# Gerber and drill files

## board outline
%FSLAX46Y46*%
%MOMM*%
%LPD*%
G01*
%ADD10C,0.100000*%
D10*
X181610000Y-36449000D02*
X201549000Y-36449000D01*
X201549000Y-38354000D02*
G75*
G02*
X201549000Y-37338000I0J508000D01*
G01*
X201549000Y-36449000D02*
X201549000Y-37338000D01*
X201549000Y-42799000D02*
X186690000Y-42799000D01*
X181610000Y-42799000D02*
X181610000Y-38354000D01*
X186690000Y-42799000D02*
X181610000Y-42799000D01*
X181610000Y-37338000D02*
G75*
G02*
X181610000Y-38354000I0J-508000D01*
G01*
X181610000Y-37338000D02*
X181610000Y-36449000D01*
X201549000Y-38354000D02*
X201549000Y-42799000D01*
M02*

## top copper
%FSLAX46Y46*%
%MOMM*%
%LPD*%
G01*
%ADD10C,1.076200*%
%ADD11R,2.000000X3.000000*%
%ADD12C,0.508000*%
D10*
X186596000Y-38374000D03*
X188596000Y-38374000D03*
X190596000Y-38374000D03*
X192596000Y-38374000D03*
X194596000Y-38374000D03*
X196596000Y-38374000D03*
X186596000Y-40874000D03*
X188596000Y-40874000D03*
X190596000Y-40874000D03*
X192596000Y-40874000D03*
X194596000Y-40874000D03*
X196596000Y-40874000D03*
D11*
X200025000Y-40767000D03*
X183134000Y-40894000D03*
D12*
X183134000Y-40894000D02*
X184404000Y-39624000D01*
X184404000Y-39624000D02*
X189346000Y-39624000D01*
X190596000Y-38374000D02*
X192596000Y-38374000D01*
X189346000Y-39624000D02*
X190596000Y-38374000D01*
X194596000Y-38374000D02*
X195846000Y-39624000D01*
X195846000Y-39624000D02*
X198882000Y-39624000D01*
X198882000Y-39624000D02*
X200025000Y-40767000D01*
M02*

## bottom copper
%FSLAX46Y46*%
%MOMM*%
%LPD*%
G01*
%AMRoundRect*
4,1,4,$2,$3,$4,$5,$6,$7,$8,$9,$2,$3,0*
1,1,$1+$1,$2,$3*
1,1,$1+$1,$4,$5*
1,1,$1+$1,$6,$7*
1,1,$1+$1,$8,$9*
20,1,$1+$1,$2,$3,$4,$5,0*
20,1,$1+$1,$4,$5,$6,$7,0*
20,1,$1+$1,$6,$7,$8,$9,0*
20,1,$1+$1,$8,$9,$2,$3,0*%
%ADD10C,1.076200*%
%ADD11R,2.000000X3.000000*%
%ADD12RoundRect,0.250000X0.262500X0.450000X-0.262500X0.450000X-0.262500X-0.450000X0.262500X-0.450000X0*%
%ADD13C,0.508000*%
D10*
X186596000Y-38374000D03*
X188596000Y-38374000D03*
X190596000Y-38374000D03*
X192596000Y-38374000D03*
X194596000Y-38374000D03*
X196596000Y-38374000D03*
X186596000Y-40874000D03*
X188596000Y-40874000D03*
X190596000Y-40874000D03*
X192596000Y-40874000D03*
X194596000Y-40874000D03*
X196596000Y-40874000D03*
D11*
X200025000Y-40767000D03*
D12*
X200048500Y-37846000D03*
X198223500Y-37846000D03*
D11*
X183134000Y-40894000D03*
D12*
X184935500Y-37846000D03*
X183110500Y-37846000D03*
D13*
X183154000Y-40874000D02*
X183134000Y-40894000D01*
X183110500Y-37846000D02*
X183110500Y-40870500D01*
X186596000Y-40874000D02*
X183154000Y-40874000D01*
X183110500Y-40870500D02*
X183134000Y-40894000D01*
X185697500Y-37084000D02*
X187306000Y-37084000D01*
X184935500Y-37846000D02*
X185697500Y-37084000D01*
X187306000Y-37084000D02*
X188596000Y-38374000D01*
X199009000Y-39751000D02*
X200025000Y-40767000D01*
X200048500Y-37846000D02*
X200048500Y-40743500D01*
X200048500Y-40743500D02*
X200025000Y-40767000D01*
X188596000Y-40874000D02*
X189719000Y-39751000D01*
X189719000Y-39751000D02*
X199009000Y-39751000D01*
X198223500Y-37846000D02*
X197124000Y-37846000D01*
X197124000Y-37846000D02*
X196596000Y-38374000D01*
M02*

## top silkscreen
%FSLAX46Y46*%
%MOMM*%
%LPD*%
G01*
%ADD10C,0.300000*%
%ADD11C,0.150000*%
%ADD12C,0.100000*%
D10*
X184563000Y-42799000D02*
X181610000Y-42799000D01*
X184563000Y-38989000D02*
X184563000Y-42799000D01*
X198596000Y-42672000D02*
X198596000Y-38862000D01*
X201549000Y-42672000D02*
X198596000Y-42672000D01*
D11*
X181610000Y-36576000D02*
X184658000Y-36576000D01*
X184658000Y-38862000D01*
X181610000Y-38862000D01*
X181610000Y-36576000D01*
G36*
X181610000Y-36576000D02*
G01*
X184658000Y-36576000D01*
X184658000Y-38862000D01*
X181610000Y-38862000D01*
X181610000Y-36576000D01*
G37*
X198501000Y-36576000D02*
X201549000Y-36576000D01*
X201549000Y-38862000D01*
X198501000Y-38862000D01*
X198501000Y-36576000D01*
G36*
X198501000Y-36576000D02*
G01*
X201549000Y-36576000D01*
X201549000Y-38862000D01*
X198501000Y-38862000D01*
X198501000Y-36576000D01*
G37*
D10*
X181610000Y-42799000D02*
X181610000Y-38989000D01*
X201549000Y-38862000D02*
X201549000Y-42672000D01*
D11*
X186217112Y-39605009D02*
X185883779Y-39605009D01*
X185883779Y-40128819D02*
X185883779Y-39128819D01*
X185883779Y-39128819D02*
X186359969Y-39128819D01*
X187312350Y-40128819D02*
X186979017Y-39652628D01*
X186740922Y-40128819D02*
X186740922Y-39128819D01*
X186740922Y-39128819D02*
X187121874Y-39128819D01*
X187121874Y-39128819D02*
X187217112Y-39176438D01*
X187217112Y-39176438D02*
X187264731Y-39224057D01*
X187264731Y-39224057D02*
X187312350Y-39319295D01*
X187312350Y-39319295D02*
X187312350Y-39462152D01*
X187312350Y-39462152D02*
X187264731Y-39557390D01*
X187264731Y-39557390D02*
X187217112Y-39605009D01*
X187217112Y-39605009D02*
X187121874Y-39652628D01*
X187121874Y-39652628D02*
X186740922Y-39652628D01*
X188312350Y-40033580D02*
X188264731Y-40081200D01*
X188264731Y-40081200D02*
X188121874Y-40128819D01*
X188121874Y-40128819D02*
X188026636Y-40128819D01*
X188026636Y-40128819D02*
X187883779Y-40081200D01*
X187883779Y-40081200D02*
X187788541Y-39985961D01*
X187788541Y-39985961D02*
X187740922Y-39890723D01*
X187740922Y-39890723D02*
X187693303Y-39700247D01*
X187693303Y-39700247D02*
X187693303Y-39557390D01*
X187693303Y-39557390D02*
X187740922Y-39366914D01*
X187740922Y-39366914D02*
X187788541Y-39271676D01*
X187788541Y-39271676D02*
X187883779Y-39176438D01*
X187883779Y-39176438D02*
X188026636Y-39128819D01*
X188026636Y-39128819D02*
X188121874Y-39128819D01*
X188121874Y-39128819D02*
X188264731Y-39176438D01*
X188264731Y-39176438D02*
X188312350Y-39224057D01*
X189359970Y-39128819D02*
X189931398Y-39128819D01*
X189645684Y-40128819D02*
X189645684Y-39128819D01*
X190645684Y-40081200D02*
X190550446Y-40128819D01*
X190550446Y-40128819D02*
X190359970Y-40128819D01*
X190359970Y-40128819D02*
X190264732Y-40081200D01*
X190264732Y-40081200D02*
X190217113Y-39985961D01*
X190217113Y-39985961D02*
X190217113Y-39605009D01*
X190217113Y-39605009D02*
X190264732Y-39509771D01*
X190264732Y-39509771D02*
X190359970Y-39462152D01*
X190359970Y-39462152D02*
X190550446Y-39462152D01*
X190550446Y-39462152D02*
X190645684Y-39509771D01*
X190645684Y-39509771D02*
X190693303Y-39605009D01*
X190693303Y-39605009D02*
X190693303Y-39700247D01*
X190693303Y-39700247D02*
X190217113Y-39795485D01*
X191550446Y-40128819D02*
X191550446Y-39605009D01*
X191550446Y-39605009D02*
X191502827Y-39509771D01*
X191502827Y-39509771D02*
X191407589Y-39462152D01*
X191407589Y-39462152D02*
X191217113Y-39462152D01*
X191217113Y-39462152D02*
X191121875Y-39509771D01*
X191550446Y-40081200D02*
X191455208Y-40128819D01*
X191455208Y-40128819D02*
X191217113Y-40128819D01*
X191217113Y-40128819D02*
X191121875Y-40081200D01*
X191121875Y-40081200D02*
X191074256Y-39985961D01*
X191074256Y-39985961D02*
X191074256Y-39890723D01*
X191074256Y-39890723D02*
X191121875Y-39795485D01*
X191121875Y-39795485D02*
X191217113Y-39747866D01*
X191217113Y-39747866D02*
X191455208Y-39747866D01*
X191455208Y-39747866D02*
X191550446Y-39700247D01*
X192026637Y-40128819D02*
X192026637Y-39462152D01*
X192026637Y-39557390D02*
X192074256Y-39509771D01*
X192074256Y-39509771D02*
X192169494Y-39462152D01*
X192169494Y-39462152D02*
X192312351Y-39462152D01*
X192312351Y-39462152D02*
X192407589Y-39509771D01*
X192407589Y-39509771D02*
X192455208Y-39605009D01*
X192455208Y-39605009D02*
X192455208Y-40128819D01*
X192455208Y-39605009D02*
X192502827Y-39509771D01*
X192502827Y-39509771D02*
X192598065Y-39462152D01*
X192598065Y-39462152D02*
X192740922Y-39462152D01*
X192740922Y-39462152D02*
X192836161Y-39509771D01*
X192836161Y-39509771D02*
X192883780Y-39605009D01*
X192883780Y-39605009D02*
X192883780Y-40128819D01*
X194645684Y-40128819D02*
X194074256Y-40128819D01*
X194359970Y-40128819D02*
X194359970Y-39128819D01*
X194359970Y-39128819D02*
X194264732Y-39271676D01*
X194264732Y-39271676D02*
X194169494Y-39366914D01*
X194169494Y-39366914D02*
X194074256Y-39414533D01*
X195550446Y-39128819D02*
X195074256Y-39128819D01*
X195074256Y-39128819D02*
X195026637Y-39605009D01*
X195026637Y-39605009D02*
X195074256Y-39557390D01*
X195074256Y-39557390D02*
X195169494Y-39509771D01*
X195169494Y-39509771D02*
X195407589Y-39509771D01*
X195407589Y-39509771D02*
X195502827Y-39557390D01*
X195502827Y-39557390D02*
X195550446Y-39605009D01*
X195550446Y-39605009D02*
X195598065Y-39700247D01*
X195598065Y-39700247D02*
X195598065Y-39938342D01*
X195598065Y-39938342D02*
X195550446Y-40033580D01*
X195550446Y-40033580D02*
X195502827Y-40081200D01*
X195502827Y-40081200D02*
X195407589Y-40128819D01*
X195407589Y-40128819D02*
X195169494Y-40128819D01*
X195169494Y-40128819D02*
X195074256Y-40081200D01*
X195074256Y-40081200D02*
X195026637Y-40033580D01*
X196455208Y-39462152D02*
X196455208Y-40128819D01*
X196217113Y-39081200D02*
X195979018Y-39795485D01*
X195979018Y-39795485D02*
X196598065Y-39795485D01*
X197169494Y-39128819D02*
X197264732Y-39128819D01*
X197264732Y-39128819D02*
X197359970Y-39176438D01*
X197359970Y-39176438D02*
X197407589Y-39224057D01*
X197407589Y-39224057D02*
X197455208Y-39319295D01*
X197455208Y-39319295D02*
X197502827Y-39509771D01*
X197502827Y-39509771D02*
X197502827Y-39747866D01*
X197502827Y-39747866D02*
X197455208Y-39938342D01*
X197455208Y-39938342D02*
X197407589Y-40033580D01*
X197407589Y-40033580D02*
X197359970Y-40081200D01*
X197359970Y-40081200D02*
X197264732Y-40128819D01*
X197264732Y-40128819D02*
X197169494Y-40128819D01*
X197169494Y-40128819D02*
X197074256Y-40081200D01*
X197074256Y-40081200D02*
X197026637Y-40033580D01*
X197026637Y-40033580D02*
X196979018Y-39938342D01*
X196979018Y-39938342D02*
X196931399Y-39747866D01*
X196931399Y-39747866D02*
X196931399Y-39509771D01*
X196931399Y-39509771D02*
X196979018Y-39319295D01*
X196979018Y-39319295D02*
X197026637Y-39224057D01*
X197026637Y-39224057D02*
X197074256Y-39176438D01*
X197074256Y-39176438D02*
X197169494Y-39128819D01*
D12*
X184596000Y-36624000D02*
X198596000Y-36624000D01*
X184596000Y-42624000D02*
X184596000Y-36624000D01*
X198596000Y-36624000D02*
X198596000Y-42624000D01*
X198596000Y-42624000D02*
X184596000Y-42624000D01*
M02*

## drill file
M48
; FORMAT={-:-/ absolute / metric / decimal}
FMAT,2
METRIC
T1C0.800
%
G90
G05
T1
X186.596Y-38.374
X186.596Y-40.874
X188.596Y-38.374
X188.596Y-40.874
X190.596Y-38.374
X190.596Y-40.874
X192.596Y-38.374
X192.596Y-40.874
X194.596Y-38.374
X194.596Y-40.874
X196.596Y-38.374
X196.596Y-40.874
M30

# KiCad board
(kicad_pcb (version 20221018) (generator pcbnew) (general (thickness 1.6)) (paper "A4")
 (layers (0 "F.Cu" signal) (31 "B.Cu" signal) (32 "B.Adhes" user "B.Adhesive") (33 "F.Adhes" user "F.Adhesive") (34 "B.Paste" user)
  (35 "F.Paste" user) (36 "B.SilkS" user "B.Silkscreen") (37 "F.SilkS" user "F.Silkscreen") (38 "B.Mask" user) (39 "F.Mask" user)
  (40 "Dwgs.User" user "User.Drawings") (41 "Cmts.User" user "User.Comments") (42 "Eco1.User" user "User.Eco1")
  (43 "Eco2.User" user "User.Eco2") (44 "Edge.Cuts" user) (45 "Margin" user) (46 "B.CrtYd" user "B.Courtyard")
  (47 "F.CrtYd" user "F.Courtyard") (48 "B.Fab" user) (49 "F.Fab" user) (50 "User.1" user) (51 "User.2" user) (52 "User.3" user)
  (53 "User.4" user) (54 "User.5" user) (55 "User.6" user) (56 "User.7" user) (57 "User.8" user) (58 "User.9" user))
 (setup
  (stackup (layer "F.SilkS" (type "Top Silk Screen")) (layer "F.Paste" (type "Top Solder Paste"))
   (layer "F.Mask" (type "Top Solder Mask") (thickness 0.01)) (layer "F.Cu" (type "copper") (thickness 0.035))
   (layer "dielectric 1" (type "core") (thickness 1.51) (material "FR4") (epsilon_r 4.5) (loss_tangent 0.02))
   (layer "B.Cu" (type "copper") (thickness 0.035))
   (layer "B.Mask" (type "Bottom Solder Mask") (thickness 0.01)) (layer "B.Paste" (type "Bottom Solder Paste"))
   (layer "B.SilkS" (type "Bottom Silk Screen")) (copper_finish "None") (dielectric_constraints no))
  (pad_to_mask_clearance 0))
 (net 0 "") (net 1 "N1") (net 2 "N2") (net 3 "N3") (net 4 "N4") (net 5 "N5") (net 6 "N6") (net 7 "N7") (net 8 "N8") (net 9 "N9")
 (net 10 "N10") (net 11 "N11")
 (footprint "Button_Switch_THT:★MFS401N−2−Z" (layer "F.Cu") (at 191.596 39.624)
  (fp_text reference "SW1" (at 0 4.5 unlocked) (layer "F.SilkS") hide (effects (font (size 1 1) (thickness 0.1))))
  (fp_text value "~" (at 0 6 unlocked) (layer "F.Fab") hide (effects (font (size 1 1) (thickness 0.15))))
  (fp_line (start -7 -3) (end 7 -3) (stroke (width 0.1) (type default)) (layer "F.SilkS"))
  (fp_line (start -7 3) (end -7 -3) (stroke (width 0.1) (type default)) (layer "F.SilkS"))
  (fp_line (start 7 -3) (end 7 3) (stroke (width 0.1) (type default)) (layer "F.SilkS"))
  (fp_line (start 7 3) (end -7 3) (stroke (width 0.1) (type default)) (layer "F.SilkS"))
  (pad "1" thru_hole circle (at -5 -1.25) (size 1.0762 1.0762) (drill 0.8) (layers "*.Cu" "*.Mask") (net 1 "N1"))
  (pad "2" thru_hole circle (at -3 -1.25) (size 1.0762 1.0762) (drill 0.8) (layers "*.Cu" "*.Mask") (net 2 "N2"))
  (pad "3" thru_hole circle (at -1 -1.25) (size 1.0762 1.0762) (drill 0.8) (layers "*.Cu" "*.Mask") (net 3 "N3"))
  (pad "4" thru_hole circle (at 1 -1.25) (size 1.0762 1.0762) (drill 0.8) (layers "*.Cu" "*.Mask") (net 3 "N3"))
  (pad "5" thru_hole circle (at 3 -1.25) (size 1.0762 1.0762) (drill 0.8) (layers "*.Cu" "*.Mask") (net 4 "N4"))
  (pad "6" thru_hole circle (at 5 -1.25) (size 1.0762 1.0762) (drill 0.8) (layers "*.Cu" "*.Mask") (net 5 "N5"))
  (pad "7" thru_hole circle (at -5 1.25) (size 1.0762 1.0762) (drill 0.8) (layers "*.Cu" "*.Mask") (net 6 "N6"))
  (pad "8" thru_hole circle (at -3 1.25) (size 1.0762 1.0762) (drill 0.8) (layers "*.Cu" "*.Mask") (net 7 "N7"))
  (pad "9" thru_hole circle (at -1 1.25) (size 1.0762 1.0762) (drill 0.8) (layers "*.Cu" "*.Mask") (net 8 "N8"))
  (pad "10" thru_hole circle (at 1 1.25) (size 1.0762 1.0762) (drill 0.8) (layers "*.Cu" "*.Mask") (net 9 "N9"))
  (pad "11" thru_hole circle (at 3 1.25) (size 1.0762 1.0762) (drill 0.8) (layers "*.Cu" "*.Mask") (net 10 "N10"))
  (pad "12" thru_hole circle (at 5 1.25) (size 1.0762 1.0762) (drill 0.8) (layers "*.Cu" "*.Mask") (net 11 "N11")))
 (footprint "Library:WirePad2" (layer "B.Cu") (at 200.025 40.767)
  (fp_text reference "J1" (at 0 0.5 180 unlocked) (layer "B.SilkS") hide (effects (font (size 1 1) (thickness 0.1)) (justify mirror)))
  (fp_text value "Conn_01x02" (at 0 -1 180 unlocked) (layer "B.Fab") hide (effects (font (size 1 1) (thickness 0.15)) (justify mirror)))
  (pad "1" smd rect (at 0 0 180) (size 2 3) (layers "B.Cu" "B.Paste" "B.Mask") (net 7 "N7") (thermal_bridge_angle 45))
  (pad "2" smd rect (at 0 0 90) (size 3 2) (layers "F.Cu" "F.Paste" "F.Mask") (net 4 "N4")))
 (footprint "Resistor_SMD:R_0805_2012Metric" (layer "B.Cu") (at 199.136 37.846 180)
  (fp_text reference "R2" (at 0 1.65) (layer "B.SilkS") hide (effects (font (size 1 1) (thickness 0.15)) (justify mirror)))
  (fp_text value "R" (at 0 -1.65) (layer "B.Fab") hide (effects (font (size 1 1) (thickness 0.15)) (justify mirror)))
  (pad "1" smd roundrect (at -0.9125 0 180) (size 1.025 1.4) (layers "B.Cu" "B.Paste" "B.Mask") (roundrect_rratio 0.243902) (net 7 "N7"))
  (pad "2" smd roundrect (at 0.9125 0 180) (size 1.025 1.4) (layers "B.Cu" "B.Paste" "B.Mask") (roundrect_rratio 0.243902) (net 5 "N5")))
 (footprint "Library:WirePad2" (layer "B.Cu") (at 183.134 40.894)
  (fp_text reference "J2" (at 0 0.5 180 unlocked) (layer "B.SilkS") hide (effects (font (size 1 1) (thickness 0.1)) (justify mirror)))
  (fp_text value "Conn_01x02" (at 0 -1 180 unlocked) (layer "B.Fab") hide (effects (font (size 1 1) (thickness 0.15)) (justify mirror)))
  (pad "1" smd rect (at 0 0 180) (size 2 3) (layers "B.Cu" "B.Paste" "B.Mask") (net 6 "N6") (thermal_bridge_angle 45))
  (pad "2" smd rect (at 0 0 90) (size 3 2) (layers "F.Cu" "F.Paste" "F.Mask") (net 3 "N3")))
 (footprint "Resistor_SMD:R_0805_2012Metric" (layer "B.Cu") (at 184.023 37.846 180)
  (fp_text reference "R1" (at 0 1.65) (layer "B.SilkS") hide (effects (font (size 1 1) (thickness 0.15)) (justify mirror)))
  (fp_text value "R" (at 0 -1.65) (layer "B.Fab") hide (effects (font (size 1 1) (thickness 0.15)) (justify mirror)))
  (pad "1" smd roundrect (at -0.9125 0 180) (size 1.025 1.4) (layers "B.Cu" "B.Paste" "B.Mask") (roundrect_rratio 0.243902) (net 2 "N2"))
  (pad "2" smd roundrect (at 0.9125 0 180) (size 1.025 1.4) (layers "B.Cu" "B.Paste" "B.Mask") (roundrect_rratio 0.243902) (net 6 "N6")))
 (gr_line (start 184.563 42.799) (end 181.61 42.799) (stroke (width 0.3) (type solid)) (layer "F.SilkS"))
 (gr_line (start 184.563 38.989) (end 184.563 42.799) (stroke (width 0.3) (type solid)) (layer "F.SilkS"))
 (gr_line (start 198.596 42.672) (end 198.596 38.862) (stroke (width 0.3) (type solid)) (layer "F.SilkS"))
 (gr_line (start 201.549 42.672) (end 198.596 42.672) (stroke (width 0.3) (type solid)) (layer "F.SilkS"))
 (gr_rect (start 181.61 36.576) (end 184.658 38.862) (stroke (width 0.15) (type solid)) (fill solid) (layer "F.SilkS"))
 (gr_rect (start 198.501 36.576) (end 201.549 38.862) (stroke (width 0.15) (type solid)) (fill solid) (layer "F.SilkS"))
 (gr_line (start 181.61 42.799) (end 181.61 38.989) (stroke (width 0.3) (type solid)) (layer "F.SilkS"))
 (gr_line (start 201.549 38.862) (end 201.549 42.672) (stroke (width 0.3) (type solid)) (layer "F.SilkS"))
 (gr_line (start 181.61 36.449) (end 201.549 36.449) (stroke (width 0.1) (type default)) (layer "Edge.Cuts"))
 (gr_arc (start 201.549 38.354) (mid 201.041 37.846) (end 201.549 37.338) (stroke (width 0.1) (type default)) (layer "Edge.Cuts"))
 (gr_line (start 201.549 36.449) (end 201.549 37.338) (stroke (width 0.1) (type default)) (layer "Edge.Cuts"))
 (gr_line (start 201.549 42.799) (end 186.69 42.799) (stroke (width 0.1) (type default)) (layer "Edge.Cuts"))
 (gr_line (start 181.61 42.799) (end 181.61 38.354) (stroke (width 0.1) (type default)) (layer "Edge.Cuts"))
 (gr_line (start 186.69 42.799) (end 181.61 42.799) (stroke (width 0.1) (type default)) (layer "Edge.Cuts"))
 (gr_arc (start 181.61 37.338) (mid 182.118 37.846) (end 181.61 38.354) (stroke (width 0.1) (type default)) (layer "Edge.Cuts"))
 (gr_line (start 181.61 37.338) (end 181.61 36.449) (stroke (width 0.1) (type default)) (layer "Edge.Cuts"))
 (gr_line (start 201.549 38.354) (end 201.549 42.799) (stroke (width 0.1) (type default)) (layer "Edge.Cuts"))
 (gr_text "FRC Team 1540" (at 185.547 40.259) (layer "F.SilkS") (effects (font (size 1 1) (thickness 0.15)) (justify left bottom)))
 (segment (start 183.154 40.874) (end 183.134 40.894) (width 0.508) (layer "B.Cu") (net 6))
 (segment (start 183.1105 37.846) (end 183.1105 40.8705) (width 0.508) (layer "B.Cu") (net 6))
 (segment (start 186.596 40.874) (end 183.154 40.874) (width 0.508) (layer "B.Cu") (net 6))
 (segment (start 183.1105 40.8705) (end 183.134 40.894) (width 0.508) (layer "B.Cu") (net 6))
 (segment (start 183.134 40.894) (end 184.404 39.624) (width 0.508) (layer "F.Cu") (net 3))
 (segment (start 184.404 39.624) (end 189.346 39.624) (width 0.508) (layer "F.Cu") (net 3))
 (segment (start 190.596 38.374) (end 192.596 38.374) (width 0.508) (layer "F.Cu") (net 3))
 (segment (start 189.346 39.624) (end 190.596 38.374) (width 0.508) (layer "F.Cu") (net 3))
 (segment (start 185.6975 37.084) (end 187.306 37.084) (width 0.508) (layer "B.Cu") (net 2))
 (segment (start 184.9355 37.846) (end 185.6975 37.084) (width 0.508) (layer "B.Cu") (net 2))
 (segment (start 187.306 37.084) (end 188.596 38.374) (width 0.508) (layer "B.Cu") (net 2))
 (segment (start 194.596 38.374) (end 195.846 39.624) (width 0.508) (layer "F.Cu") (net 4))
 (segment (start 195.846 39.624) (end 198.882 39.624) (width 0.508) (layer "F.Cu") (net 4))
 (segment (start 198.882 39.624) (end 200.025 40.767) (width 0.508) (layer "F.Cu") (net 4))
 (segment (start 199.009 39.751) (end 200.025 40.767) (width 0.508) (layer "B.Cu") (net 7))
 (segment (start 200.0485 37.846) (end 200.0485 40.7435) (width 0.508) (layer "B.Cu") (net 7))
 (segment (start 200.0485 40.7435) (end 200.025 40.767) (width 0.508) (layer "B.Cu") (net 7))
 (segment (start 188.596 40.874) (end 189.719 39.751) (width 0.508) (layer "B.Cu") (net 7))
 (segment (start 189.719 39.751) (end 199.009 39.751) (width 0.508) (layer "B.Cu") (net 7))
 (segment (start 198.2235 37.846) (end 197.124 37.846) (width 0.508) (layer "B.Cu") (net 5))
 (segment (start 197.124 37.846) (end 196.596 38.374) (width 0.508) (layer "B.Cu") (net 5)))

